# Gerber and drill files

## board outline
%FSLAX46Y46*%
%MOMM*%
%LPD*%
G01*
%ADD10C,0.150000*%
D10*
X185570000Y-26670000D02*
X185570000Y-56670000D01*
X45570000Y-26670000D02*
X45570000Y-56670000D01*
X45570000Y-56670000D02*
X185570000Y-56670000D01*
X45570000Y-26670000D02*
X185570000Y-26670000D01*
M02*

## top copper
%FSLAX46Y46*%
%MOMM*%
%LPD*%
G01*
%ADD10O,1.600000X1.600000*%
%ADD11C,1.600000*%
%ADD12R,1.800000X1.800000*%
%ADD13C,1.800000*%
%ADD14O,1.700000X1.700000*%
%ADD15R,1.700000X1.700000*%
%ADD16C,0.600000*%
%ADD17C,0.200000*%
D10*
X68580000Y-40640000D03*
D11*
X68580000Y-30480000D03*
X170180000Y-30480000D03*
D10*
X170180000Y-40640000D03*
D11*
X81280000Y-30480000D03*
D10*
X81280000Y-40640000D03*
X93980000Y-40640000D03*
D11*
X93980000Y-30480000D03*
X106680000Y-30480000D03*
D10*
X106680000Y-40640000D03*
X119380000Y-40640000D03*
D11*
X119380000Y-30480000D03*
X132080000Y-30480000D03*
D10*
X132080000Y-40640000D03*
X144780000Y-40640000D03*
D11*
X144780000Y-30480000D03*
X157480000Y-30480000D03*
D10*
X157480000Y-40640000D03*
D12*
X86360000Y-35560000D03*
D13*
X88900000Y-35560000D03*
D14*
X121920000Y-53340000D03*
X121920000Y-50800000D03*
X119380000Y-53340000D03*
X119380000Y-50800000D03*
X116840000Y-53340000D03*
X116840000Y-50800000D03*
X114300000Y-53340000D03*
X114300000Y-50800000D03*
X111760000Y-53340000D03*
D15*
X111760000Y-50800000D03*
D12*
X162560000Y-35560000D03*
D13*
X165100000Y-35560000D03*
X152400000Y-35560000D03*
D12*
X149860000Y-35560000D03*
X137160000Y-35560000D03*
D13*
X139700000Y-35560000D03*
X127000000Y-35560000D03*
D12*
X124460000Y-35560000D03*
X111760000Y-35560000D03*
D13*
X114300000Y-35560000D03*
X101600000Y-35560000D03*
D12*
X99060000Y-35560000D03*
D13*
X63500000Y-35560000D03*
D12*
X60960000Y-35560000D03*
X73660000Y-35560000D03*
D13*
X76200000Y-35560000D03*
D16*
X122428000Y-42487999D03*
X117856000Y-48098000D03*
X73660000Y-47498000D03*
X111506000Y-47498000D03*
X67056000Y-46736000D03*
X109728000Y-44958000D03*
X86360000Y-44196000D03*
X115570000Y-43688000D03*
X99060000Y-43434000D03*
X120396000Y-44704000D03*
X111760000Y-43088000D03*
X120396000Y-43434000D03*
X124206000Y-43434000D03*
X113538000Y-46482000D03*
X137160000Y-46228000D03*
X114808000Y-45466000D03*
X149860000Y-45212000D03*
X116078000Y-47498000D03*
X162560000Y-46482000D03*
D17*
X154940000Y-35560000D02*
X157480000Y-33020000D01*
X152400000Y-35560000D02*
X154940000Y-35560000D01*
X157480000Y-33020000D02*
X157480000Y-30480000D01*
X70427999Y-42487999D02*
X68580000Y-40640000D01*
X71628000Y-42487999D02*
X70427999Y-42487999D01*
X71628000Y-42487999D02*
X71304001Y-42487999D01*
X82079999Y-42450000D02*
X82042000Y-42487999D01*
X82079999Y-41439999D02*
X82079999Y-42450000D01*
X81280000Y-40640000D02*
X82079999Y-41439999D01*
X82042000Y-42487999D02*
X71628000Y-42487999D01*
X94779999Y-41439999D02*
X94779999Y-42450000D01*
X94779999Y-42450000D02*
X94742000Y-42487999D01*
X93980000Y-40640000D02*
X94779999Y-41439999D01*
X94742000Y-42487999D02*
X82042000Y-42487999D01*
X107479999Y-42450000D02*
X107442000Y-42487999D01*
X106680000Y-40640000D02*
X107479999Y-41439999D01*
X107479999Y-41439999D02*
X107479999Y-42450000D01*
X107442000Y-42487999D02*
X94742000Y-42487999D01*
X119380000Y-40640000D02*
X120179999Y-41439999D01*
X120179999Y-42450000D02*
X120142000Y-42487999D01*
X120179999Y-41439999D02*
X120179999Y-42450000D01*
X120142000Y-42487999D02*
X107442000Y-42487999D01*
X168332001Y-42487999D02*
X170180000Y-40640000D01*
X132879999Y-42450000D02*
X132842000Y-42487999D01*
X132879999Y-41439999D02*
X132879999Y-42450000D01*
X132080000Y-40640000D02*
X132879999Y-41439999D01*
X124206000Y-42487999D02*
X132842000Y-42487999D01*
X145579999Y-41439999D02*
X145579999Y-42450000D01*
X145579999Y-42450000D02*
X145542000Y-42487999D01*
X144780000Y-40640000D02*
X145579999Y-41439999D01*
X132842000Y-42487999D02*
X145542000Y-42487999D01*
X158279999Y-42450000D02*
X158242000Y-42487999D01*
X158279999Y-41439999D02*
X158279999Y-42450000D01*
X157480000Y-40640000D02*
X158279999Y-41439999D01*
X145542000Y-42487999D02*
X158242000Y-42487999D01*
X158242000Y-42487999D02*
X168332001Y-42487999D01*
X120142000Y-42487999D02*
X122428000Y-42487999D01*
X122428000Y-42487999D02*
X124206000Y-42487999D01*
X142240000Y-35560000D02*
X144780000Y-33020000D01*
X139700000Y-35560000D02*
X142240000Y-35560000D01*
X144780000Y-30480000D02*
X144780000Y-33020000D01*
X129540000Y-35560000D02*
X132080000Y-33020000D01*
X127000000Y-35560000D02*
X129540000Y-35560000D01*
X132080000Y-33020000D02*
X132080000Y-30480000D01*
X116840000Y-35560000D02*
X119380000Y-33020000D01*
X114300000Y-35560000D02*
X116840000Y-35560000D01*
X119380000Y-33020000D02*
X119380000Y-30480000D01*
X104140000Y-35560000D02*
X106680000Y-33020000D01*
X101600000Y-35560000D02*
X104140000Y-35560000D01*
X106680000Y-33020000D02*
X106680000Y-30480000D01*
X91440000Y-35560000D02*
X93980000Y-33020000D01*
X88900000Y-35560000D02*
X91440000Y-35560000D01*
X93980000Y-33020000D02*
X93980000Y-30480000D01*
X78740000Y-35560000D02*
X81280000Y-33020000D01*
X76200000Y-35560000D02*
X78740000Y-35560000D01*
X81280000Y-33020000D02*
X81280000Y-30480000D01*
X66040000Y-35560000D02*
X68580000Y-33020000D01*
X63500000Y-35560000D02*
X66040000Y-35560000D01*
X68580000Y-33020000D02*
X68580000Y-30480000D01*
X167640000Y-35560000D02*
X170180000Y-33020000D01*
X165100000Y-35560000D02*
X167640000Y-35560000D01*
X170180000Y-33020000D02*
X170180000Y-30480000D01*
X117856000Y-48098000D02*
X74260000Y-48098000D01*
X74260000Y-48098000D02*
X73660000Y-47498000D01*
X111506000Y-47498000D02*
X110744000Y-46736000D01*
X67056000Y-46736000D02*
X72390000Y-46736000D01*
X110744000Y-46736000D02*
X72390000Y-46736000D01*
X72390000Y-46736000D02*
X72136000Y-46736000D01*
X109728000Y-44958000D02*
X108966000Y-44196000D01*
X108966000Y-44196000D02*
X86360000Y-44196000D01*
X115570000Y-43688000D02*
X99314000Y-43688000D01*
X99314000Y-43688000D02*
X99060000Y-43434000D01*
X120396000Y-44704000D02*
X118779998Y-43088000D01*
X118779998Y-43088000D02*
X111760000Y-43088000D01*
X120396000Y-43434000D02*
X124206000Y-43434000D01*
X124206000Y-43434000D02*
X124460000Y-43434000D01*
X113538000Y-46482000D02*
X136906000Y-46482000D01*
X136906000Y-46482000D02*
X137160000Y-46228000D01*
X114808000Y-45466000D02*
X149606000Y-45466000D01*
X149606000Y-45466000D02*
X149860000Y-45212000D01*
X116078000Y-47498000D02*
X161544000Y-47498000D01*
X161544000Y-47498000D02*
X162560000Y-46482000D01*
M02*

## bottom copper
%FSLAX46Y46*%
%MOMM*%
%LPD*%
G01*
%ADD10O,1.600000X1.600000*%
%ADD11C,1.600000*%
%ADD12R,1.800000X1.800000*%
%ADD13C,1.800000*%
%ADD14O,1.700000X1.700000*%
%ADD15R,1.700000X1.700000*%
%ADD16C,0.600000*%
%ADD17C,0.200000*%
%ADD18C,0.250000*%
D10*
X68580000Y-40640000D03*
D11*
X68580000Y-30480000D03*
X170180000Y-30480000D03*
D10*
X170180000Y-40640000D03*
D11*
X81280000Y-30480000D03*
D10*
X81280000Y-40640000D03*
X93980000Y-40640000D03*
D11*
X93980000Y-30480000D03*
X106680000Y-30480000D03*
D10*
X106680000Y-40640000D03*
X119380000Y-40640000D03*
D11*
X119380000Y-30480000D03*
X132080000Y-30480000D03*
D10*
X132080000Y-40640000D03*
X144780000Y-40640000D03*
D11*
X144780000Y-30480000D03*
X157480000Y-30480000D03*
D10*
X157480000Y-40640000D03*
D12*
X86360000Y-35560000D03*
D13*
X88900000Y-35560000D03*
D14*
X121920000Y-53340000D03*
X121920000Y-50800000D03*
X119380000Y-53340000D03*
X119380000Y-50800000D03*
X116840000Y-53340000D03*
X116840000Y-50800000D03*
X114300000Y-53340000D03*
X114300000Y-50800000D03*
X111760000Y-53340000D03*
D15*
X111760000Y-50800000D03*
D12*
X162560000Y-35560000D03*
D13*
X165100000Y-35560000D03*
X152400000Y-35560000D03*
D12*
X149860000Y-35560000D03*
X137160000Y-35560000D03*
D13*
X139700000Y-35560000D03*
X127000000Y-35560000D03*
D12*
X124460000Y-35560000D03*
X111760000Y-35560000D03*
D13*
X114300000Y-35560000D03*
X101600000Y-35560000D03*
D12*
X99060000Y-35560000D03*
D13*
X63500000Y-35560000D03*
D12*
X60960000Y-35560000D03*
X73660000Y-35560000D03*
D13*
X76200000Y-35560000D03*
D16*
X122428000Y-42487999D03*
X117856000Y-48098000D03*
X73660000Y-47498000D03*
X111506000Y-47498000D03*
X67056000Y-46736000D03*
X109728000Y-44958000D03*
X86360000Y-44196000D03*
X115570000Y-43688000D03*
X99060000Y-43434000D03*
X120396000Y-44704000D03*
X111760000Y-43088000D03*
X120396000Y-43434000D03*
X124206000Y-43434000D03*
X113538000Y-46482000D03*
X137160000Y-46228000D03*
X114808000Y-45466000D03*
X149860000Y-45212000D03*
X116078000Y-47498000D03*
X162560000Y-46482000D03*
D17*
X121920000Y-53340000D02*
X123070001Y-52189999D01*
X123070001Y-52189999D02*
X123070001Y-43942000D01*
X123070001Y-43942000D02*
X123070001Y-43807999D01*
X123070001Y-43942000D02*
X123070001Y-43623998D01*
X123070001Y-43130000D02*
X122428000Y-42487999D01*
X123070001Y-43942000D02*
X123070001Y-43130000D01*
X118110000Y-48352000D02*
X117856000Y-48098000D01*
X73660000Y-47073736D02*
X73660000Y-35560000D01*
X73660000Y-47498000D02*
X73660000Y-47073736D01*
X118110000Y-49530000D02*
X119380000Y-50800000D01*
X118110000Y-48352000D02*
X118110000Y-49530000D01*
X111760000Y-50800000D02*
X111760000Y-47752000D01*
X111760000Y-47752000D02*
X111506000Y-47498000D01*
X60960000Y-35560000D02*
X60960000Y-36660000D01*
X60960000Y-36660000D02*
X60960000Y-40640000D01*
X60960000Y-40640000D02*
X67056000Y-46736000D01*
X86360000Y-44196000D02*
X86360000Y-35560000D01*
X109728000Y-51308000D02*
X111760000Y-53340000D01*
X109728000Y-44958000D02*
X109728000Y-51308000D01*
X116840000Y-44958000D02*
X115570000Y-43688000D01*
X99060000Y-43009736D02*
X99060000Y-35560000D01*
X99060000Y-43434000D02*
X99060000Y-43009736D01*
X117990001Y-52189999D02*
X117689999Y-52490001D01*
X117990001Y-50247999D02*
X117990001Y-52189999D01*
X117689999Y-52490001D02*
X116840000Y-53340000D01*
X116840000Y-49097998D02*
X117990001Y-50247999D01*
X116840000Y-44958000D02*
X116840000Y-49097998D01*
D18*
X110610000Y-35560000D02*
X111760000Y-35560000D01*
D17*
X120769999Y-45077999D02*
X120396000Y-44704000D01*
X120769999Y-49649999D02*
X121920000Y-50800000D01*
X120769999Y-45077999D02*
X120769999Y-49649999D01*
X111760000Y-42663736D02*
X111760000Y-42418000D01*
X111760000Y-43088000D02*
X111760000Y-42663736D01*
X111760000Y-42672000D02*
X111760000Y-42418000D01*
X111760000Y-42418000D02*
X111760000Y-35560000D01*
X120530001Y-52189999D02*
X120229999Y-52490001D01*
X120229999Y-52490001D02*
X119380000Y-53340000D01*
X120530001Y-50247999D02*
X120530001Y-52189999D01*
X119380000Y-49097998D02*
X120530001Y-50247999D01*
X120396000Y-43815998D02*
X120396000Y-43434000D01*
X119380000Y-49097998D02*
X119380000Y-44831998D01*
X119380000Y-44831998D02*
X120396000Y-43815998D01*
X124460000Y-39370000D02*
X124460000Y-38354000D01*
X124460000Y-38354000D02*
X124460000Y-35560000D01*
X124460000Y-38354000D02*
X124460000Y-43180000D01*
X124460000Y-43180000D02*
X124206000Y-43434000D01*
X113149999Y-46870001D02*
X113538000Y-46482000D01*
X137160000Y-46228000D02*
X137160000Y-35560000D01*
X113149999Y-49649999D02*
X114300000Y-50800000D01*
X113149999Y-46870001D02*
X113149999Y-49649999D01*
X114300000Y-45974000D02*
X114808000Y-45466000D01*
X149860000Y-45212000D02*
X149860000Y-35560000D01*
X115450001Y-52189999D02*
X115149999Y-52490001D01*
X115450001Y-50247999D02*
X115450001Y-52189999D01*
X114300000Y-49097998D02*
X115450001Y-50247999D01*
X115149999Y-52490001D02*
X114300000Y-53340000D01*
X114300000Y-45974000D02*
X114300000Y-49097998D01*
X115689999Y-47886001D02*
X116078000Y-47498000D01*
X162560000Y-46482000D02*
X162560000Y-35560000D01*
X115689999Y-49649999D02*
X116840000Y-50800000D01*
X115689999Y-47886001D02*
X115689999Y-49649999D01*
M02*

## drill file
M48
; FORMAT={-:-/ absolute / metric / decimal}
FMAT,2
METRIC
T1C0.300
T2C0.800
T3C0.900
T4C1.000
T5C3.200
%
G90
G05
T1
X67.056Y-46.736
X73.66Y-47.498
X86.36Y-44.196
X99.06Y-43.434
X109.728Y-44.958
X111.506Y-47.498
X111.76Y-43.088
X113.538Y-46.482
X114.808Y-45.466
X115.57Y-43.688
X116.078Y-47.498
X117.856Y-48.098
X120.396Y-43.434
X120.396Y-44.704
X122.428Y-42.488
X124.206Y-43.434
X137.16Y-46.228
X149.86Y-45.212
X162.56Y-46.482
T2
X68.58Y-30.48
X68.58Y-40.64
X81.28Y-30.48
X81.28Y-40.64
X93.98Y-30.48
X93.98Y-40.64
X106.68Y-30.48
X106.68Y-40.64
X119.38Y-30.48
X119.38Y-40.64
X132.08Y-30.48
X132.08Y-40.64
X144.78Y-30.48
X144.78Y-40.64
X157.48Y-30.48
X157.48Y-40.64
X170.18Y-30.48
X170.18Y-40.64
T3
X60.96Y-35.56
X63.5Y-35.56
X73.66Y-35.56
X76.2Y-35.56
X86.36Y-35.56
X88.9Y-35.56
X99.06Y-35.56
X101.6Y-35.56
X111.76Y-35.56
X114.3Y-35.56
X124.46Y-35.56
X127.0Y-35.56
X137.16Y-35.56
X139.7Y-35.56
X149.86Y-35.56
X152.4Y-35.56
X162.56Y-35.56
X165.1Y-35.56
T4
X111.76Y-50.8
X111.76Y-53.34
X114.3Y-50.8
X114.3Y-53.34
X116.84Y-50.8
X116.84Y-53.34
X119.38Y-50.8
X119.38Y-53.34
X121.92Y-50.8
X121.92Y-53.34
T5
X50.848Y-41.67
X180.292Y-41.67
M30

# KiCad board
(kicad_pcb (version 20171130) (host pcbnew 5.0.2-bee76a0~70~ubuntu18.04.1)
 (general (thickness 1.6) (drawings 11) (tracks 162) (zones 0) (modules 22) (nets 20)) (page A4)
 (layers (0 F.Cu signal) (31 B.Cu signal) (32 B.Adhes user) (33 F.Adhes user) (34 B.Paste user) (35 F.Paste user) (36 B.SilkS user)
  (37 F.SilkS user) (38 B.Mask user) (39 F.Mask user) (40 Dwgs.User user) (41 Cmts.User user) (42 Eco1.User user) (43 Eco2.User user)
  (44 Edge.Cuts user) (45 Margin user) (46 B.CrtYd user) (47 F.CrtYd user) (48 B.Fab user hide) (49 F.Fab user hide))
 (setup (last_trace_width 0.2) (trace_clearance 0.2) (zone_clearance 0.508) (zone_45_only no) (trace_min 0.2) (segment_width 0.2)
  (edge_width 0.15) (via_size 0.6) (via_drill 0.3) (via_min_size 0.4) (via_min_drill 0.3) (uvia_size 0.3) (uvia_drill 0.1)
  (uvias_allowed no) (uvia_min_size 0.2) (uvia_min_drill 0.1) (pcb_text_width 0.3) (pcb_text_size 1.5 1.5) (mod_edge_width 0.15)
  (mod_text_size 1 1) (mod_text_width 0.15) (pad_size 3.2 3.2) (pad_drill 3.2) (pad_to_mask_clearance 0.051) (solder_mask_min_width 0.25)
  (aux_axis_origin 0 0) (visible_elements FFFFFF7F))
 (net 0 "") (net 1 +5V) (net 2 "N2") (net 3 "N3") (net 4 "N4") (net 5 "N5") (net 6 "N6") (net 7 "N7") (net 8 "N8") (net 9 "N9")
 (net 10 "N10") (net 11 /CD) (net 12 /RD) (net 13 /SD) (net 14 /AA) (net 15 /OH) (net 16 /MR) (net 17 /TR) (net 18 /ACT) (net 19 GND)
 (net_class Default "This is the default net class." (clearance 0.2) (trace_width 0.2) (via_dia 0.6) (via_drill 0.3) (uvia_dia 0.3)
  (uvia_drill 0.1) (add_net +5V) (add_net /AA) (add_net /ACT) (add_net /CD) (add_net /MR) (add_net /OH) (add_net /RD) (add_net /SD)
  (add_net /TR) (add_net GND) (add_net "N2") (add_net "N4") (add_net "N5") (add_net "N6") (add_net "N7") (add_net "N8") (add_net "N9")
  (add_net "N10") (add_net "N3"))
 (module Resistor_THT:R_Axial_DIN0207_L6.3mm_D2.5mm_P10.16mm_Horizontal (layer F.Cu) (at 68.58 30.48 270)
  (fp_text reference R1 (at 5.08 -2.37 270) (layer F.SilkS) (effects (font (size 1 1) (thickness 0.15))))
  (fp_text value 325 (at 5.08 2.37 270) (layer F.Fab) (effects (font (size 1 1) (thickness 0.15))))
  (pad 2 thru_hole oval (at 10.16 0 270) (size 1.6 1.6) (drill 0.8) (layers *.Cu *.Mask) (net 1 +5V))
  (pad 1 thru_hole circle (at 0 0 270) (size 1.6 1.6) (drill 0.8) (layers *.Cu *.Mask) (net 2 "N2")))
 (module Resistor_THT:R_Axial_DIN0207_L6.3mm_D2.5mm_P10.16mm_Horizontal (layer F.Cu) (at 170.18 30.48 270)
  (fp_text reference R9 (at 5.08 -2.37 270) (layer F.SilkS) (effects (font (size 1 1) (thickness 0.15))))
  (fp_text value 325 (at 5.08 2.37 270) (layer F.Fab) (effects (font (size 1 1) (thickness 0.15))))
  (pad 1 thru_hole circle (at 0 0 270) (size 1.6 1.6) (drill 0.8) (layers *.Cu *.Mask) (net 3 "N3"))
  (pad 2 thru_hole oval (at 10.16 0 270) (size 1.6 1.6) (drill 0.8) (layers *.Cu *.Mask) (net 1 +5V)))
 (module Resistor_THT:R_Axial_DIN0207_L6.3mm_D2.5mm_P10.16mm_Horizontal (layer F.Cu) (at 81.28 30.48 270)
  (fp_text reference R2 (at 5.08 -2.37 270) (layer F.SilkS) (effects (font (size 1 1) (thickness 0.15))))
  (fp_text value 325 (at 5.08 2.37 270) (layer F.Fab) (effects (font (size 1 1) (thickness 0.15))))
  (pad 1 thru_hole circle (at 0 0 270) (size 1.6 1.6) (drill 0.8) (layers *.Cu *.Mask) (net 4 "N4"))
  (pad 2 thru_hole oval (at 10.16 0 270) (size 1.6 1.6) (drill 0.8) (layers *.Cu *.Mask) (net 1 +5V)))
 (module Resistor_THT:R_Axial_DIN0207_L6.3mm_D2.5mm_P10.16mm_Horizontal (layer F.Cu) (at 93.98 30.48 270)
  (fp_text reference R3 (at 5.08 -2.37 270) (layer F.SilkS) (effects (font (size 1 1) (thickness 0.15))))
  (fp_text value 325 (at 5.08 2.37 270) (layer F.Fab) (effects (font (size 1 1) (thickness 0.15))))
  (pad 2 thru_hole oval (at 10.16 0 270) (size 1.6 1.6) (drill 0.8) (layers *.Cu *.Mask) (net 1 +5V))
  (pad 1 thru_hole circle (at 0 0 270) (size 1.6 1.6) (drill 0.8) (layers *.Cu *.Mask) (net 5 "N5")))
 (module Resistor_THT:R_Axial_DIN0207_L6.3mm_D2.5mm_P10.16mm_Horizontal (layer F.Cu) (at 106.68 30.48 270)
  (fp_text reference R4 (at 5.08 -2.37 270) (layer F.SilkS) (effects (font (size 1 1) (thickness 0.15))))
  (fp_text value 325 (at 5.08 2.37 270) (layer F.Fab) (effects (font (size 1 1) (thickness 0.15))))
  (pad 1 thru_hole circle (at 0 0 270) (size 1.6 1.6) (drill 0.8) (layers *.Cu *.Mask) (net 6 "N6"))
  (pad 2 thru_hole oval (at 10.16 0 270) (size 1.6 1.6) (drill 0.8) (layers *.Cu *.Mask) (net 1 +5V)))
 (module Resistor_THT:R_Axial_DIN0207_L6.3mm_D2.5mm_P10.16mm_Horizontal (layer F.Cu) (at 119.38 30.48 270)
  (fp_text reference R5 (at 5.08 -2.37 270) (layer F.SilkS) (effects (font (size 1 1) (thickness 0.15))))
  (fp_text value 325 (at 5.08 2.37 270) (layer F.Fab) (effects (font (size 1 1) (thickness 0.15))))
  (pad 2 thru_hole oval (at 10.16 0 270) (size 1.6 1.6) (drill 0.8) (layers *.Cu *.Mask) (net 1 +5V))
  (pad 1 thru_hole circle (at 0 0 270) (size 1.6 1.6) (drill 0.8) (layers *.Cu *.Mask) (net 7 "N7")))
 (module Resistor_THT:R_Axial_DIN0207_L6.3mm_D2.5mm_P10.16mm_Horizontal (layer F.Cu) (at 132.08 30.48 270)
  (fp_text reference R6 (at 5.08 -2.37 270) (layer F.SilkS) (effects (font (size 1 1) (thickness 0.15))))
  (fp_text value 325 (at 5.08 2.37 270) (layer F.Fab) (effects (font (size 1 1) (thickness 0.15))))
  (pad 1 thru_hole circle (at 0 0 270) (size 1.6 1.6) (drill 0.8) (layers *.Cu *.Mask) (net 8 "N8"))
  (pad 2 thru_hole oval (at 10.16 0 270) (size 1.6 1.6) (drill 0.8) (layers *.Cu *.Mask) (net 1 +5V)))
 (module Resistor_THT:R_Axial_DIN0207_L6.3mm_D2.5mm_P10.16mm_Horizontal (layer F.Cu) (at 144.78 30.48 270)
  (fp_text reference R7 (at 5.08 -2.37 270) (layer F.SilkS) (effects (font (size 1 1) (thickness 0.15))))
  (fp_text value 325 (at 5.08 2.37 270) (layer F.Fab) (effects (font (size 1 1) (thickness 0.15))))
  (pad 2 thru_hole oval (at 10.16 0 270) (size 1.6 1.6) (drill 0.8) (layers *.Cu *.Mask) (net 1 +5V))
  (pad 1 thru_hole circle (at 0 0 270) (size 1.6 1.6) (drill 0.8) (layers *.Cu *.Mask) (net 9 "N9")))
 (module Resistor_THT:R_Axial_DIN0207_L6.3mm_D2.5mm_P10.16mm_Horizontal (layer F.Cu) (at 157.48 30.48 270)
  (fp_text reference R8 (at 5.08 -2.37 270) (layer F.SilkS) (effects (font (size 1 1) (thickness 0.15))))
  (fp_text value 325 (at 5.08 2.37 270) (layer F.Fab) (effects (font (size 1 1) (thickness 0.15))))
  (pad 1 thru_hole circle (at 0 0 270) (size 1.6 1.6) (drill 0.8) (layers *.Cu *.Mask) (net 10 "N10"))
  (pad 2 thru_hole oval (at 10.16 0 270) (size 1.6 1.6) (drill 0.8) (layers *.Cu *.Mask) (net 1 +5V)))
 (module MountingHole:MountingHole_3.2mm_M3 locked (layer F.Cu) (at 180.292 41.67)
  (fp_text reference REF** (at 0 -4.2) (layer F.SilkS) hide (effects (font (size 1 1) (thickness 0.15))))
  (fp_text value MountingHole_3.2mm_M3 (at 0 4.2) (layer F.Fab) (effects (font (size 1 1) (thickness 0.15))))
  (pad 1 np_thru_hole circle (at 0 0) (size 3.2 3.2) (drill 3.2) (layers *.Cu *.Mask)))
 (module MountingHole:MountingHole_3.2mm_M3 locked (layer F.Cu) (at 50.848 41.67)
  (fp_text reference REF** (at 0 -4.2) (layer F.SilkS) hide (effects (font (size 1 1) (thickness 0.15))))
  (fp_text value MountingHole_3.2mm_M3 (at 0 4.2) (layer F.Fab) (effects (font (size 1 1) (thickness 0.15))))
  (pad 1 np_thru_hole circle (at 0 0) (size 3.2 3.2) (drill 3.2) (layers *.Cu *.Mask)))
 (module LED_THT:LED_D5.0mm (layer F.Cu) (at 86.36 35.56)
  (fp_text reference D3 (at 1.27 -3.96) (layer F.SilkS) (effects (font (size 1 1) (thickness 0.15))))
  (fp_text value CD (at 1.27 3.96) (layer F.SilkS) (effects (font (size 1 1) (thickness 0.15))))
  (pad 1 thru_hole rect (at 0 0) (size 1.8 1.8) (drill 0.9) (layers *.Cu *.Mask) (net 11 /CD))
  (pad 2 thru_hole circle (at 2.54 0) (size 1.8 1.8) (drill 0.9) (layers *.Cu *.Mask) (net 5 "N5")))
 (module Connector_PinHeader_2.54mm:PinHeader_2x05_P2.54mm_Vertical (layer B.Cu) (at 111.76 50.8 270)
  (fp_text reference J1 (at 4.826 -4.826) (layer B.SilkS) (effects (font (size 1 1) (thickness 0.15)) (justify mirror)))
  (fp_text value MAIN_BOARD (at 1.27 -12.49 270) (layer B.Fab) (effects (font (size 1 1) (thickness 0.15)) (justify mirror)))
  (pad 10 thru_hole oval (at 2.54 -10.16 270) (size 1.7 1.7) (drill 1) (layers *.Cu *.Mask) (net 1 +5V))
  (pad 9 thru_hole oval (at 0 -10.16 270) (size 1.7 1.7) (drill 1) (layers *.Cu *.Mask) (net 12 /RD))
  (pad 8 thru_hole oval (at 2.54 -7.62 270) (size 1.7 1.7) (drill 1) (layers *.Cu *.Mask) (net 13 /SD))
  (pad 7 thru_hole oval (at 0 -7.62 270) (size 1.7 1.7) (drill 1) (layers *.Cu *.Mask) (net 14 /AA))
  (pad 6 thru_hole oval (at 2.54 -5.08 270) (size 1.7 1.7) (drill 1) (layers *.Cu *.Mask) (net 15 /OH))
  (pad 5 thru_hole oval (at 0 -5.08 270) (size 1.7 1.7) (drill 1) (layers *.Cu *.Mask) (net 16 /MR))
  (pad 4 thru_hole oval (at 2.54 -2.54 270) (size 1.7 1.7) (drill 1) (layers *.Cu *.Mask) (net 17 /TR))
  (pad 3 thru_hole oval (at 0 -2.54 270) (size 1.7 1.7) (drill 1) (layers *.Cu *.Mask) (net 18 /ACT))
  (pad 2 thru_hole oval (at 2.54 0 270) (size 1.7 1.7) (drill 1) (layers *.Cu *.Mask) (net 11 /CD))
  (pad 1 thru_hole rect (at 0 0 270) (size 1.7 1.7) (drill 1) (layers *.Cu *.Mask) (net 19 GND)))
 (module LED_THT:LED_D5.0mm (layer F.Cu) (at 162.56 35.56)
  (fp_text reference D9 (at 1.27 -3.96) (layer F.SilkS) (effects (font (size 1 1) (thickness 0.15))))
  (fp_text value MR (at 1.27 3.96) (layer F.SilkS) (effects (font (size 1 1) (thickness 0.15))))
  (pad 1 thru_hole rect (at 0 0) (size 1.8 1.8) (drill 0.9) (layers *.Cu *.Mask) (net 16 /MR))
  (pad 2 thru_hole circle (at 2.54 0) (size 1.8 1.8) (drill 0.9) (layers *.Cu *.Mask) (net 3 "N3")))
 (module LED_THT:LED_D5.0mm (layer F.Cu) (at 149.86 35.56)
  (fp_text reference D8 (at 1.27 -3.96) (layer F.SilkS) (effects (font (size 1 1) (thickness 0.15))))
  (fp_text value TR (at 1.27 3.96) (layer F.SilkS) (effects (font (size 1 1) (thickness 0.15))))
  (pad 2 thru_hole circle (at 2.54 0) (size 1.8 1.8) (drill 0.9) (layers *.Cu *.Mask) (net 10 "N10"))
  (pad 1 thru_hole rect (at 0 0) (size 1.8 1.8) (drill 0.9) (layers *.Cu *.Mask) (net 17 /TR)))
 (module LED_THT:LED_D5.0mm (layer F.Cu) (at 137.16 35.56)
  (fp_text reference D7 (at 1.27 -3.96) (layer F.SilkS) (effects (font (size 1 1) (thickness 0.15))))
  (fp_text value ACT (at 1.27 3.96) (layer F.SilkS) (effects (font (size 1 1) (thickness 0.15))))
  (pad 1 thru_hole rect (at 0 0) (size 1.8 1.8) (drill 0.9) (layers *.Cu *.Mask) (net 18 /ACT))
  (pad 2 thru_hole circle (at 2.54 0) (size 1.8 1.8) (drill 0.9) (layers *.Cu *.Mask) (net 9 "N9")))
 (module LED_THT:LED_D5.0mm (layer F.Cu) (at 124.46 35.56)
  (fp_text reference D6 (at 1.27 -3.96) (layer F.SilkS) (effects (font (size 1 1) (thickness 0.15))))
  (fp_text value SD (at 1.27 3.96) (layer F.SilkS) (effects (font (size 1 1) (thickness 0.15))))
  (pad 2 thru_hole circle (at 2.54 0) (size 1.8 1.8) (drill 0.9) (layers *.Cu *.Mask) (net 8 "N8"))
  (pad 1 thru_hole rect (at 0 0) (size 1.8 1.8) (drill 0.9) (layers *.Cu *.Mask) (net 13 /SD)))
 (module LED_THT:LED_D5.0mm (layer F.Cu) (at 111.76 35.56)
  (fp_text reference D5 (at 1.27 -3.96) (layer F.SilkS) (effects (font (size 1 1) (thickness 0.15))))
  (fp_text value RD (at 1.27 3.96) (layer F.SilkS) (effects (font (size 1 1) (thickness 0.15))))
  (pad 1 thru_hole rect (at 0 0) (size 1.8 1.8) (drill 0.9) (layers *.Cu *.Mask) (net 12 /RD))
  (pad 2 thru_hole circle (at 2.54 0) (size 1.8 1.8) (drill 0.9) (layers *.Cu *.Mask) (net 7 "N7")))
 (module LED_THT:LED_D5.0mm (layer F.Cu) (at 99.06 35.56)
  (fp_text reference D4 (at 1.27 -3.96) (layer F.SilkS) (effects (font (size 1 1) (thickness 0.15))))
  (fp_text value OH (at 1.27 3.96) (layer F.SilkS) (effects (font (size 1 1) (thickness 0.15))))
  (pad 2 thru_hole circle (at 2.54 0) (size 1.8 1.8) (drill 0.9) (layers *.Cu *.Mask) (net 6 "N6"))
  (pad 1 thru_hole rect (at 0 0) (size 1.8 1.8) (drill 0.9) (layers *.Cu *.Mask) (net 15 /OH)))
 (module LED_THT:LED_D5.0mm (layer F.Cu) (at 60.96 35.56)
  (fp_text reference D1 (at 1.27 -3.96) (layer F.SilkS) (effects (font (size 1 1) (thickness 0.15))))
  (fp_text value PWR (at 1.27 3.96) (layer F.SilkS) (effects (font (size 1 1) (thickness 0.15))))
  (pad 2 thru_hole circle (at 2.54 0) (size 1.8 1.8) (drill 0.9) (layers *.Cu *.Mask) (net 2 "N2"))
  (pad 1 thru_hole rect (at 0 0) (size 1.8 1.8) (drill 0.9) (layers *.Cu *.Mask) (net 19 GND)))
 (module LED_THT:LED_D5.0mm (layer F.Cu) (at 73.66 35.56)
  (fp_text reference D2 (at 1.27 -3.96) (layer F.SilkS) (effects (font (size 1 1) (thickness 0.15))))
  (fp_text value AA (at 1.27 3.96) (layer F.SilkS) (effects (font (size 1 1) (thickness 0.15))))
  (pad 1 thru_hole rect (at 0 0) (size 1.8 1.8) (drill 0.9) (layers *.Cu *.Mask) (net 14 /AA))
  (pad 2 thru_hole circle (at 2.54 0) (size 1.8 1.8) (drill 0.9) (layers *.Cu *.Mask) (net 4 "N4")))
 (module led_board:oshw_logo (layer F.Cu) (at 51.01 50.8)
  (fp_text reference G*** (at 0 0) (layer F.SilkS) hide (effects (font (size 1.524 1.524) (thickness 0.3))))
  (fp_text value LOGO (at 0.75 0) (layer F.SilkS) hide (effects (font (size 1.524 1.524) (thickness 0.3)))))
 (gr_line (start 185.57 26.67) (end 185.57 56.67) (layer Edge.Cuts) (width 0.15))
 (gr_line (start 45.57 26.67) (end 45.57 56.67) (layer Edge.Cuts) (width 0.15))
 (gr_line (start 45.57 56.67) (end 185.57 56.67) (layer Edge.Cuts) (width 0.15))
 (gr_line (start 45.57 26.67) (end 185.57 26.67) (layer Edge.Cuts) (width 0.15))
 (segment (start 154.94 35.56) (end 157.48 33.02) (width 0.2) (layer F.Cu) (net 10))
 (segment (start 152.4 35.56) (end 154.94 35.56) (width 0.2) (layer F.Cu) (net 10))
 (segment (start 157.48 33.02) (end 157.48 30.48) (width 0.2) (layer F.Cu) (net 10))
 (segment (start 121.92 53.34) (end 123.070001 52.189999) (width 0.2) (layer B.Cu) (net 1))
 (segment (start 70.427999 42.487999) (end 68.58 40.64) (width 0.2) (layer F.Cu) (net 1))
 (segment (start 71.628 42.487999) (end 70.427999 42.487999) (width 0.2) (layer F.Cu) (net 1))
 (segment (start 71.628 42.487999) (end 71.304001 42.487999) (width 0.2) (layer F.Cu) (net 1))
 (segment (start 82.079999 42.45) (end 82.042 42.487999) (width 0.2) (layer F.Cu) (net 1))
 (segment (start 82.079999 41.439999) (end 82.079999 42.45) (width 0.2) (layer F.Cu) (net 1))
 (segment (start 81.28 40.64) (end 82.079999 41.439999) (width 0.2) (layer F.Cu) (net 1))
 (segment (start 82.042 42.487999) (end 71.628 42.487999) (width 0.2) (layer F.Cu) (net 1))
 (segment (start 94.779999 41.439999) (end 94.779999 42.45) (width 0.2) (layer F.Cu) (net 1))
 (segment (start 94.779999 42.45) (end 94.742 42.487999) (width 0.2) (layer F.Cu) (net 1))
 (segment (start 93.98 40.64) (end 94.779999 41.439999) (width 0.2) (layer F.Cu) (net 1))
 (segment (start 94.742 42.487999) (end 82.042 42.487999) (width 0.2) (layer F.Cu) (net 1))
 (segment (start 107.479999 42.45) (end 107.442 42.487999) (width 0.2) (layer F.Cu) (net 1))
 (segment (start 106.68 40.64) (end 107.479999 41.439999) (width 0.2) (layer F.Cu) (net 1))
 (segment (start 107.479999 41.439999) (end 107.479999 42.45) (width 0.2) (layer F.Cu) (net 1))
 (segment (start 107.442 42.487999) (end 94.742 42.487999) (width 0.2) (layer F.Cu) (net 1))
 (segment (start 119.38 40.64) (end 120.179999 41.439999) (width 0.2) (layer F.Cu) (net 1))
 (segment (start 120.179999 42.45) (end 120.142 42.487999) (width 0.2) (layer F.Cu) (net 1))
 (segment (start 120.179999 41.439999) (end 120.179999 42.45) (width 0.2) (layer F.Cu) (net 1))
 (segment (start 120.142 42.487999) (end 107.442 42.487999) (width 0.2) (layer F.Cu) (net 1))
 (segment (start 168.332001 42.487999) (end 170.18 40.64) (width 0.2) (layer F.Cu) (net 1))
 (segment (start 123.070001 52.189999) (end 123.070001 43.942) (width 0.2) (layer B.Cu) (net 1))
 (segment (start 123.070001 43.942) (end 123.070001 43.807999) (width 0.2) (layer B.Cu) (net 1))
 (segment (start 123.070001 43.942) (end 123.070001 43.623998) (width 0.2) (layer B.Cu) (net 1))
 (segment (start 132.879999 42.45) (end 132.842 42.487999) (width 0.2) (layer F.Cu) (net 1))
 (segment (start 132.879999 41.439999) (end 132.879999 42.45) (width 0.2) (layer F.Cu) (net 1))
 (segment (start 132.08 40.64) (end 132.879999 41.439999) (width 0.2) (layer F.Cu) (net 1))
 (segment (start 124.206 42.487999) (end 132.842 42.487999) (width 0.2) (layer F.Cu) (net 1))
 (segment (start 145.579999 41.439999) (end 145.579999 42.45) (width 0.2) (layer F.Cu) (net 1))
 (segment (start 145.579999 42.45) (end 145.542 42.487999) (width 0.2) (layer F.Cu) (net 1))
 (segment (start 144.78 40.64) (end 145.579999 41.439999) (width 0.2) (layer F.Cu) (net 1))
 (segment (start 132.842 42.487999) (end 145.542 42.487999) (width 0.2) (layer F.Cu) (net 1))
 (segment (start 158.279999 42.45) (end 158.242 42.487999) (width 0.2) (layer F.Cu) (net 1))
 (segment (start 158.279999 41.439999) (end 158.279999 42.45) (width 0.2) (layer F.Cu) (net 1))
 (segment (start 157.48 40.64) (end 158.279999 41.439999) (width 0.2) (layer F.Cu) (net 1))
 (segment (start 145.542 42.487999) (end 158.242 42.487999) (width 0.2) (layer F.Cu) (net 1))
 (segment (start 158.242 42.487999) (end 168.332001 42.487999) (width 0.2) (layer F.Cu) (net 1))
 (segment (start 123.070001 43.13) (end 122.428 42.487999) (width 0.2) (layer B.Cu) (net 1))
 (segment (start 123.070001 43.942) (end 123.070001 43.13) (width 0.2) (layer B.Cu) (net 1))
 (segment (start 120.142 42.487999) (end 122.428 42.487999) (width 0.2) (layer F.Cu) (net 1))
 (via (at 122.428 42.487999) (size 0.6) (drill 0.3) (layers F.Cu B.Cu) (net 1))
 (segment (start 122.428 42.487999) (end 124.206 42.487999) (width 0.2) (layer F.Cu) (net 1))
 (segment (start 142.24 35.56) (end 144.78 33.02) (width 0.2) (layer F.Cu) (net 9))
 (segment (start 139.7 35.56) (end 142.24 35.56) (width 0.2) (layer F.Cu) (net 9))
 (segment (start 144.78 30.48) (end 144.78 33.02) (width 0.2) (layer F.Cu) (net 9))
 (segment (start 129.54 35.56) (end 132.08 33.02) (width 0.2) (layer F.Cu) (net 8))
 (segment (start 127 35.56) (end 129.54 35.56) (width 0.2) (layer F.Cu) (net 8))
 (segment (start 132.08 33.02) (end 132.08 30.48) (width 0.2) (layer F.Cu) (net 8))
 (segment (start 116.84 35.56) (end 119.38 33.02) (width 0.2) (layer F.Cu) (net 7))
 (segment (start 114.3 35.56) (end 116.84 35.56) (width 0.2) (layer F.Cu) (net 7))
 (segment (start 119.38 33.02) (end 119.38 30.48) (width 0.2) (layer F.Cu) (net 7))
 (segment (start 104.14 35.56) (end 106.68 33.02) (width 0.2) (layer F.Cu) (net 6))
 (segment (start 101.6 35.56) (end 104.14 35.56) (width 0.2) (layer F.Cu) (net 6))
 (segment (start 106.68 33.02) (end 106.68 30.48) (width 0.2) (layer F.Cu) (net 6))
 (segment (start 91.44 35.56) (end 93.98 33.02) (width 0.2) (layer F.Cu) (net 5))
 (segment (start 88.9 35.56) (end 91.44 35.56) (width 0.2) (layer F.Cu) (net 5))
 (segment (start 93.98 33.02) (end 93.98 30.48) (width 0.2) (layer F.Cu) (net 5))
 (segment (start 78.74 35.56) (end 81.28 33.02) (width 0.2) (layer F.Cu) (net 4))
 (segment (start 76.2 35.56) (end 78.74 35.56) (width 0.2) (layer F.Cu) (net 4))
 (segment (start 81.28 33.02) (end 81.28 30.48) (width 0.2) (layer F.Cu) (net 4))
 (segment (start 66.04 35.56) (end 68.58 33.02) (width 0.2) (layer F.Cu) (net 2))
 (segment (start 63.5 35.56) (end 66.04 35.56) (width 0.2) (layer F.Cu) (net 2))
 (segment (start 68.58 33.02) (end 68.58 30.48) (width 0.2) (layer F.Cu) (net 2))
 (segment (start 167.64 35.56) (end 170.18 33.02) (width 0.2) (layer F.Cu) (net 3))
 (segment (start 165.1 35.56) (end 167.64 35.56) (width 0.2) (layer F.Cu) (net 3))
 (segment (start 170.18 33.02) (end 170.18 30.48) (width 0.2) (layer F.Cu) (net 3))
 (via (at 117.856 48.098) (size 0.6) (drill 0.3) (layers F.Cu B.Cu) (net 14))
 (segment (start 118.11 48.352) (end 117.856 48.098) (width 0.2) (layer B.Cu) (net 14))
 (via (at 73.66 47.498) (size 0.6) (drill 0.3) (layers F.Cu B.Cu) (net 14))
 (segment (start 117.856 48.098) (end 74.26 48.098) (width 0.2) (layer F.Cu) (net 14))
 (segment (start 74.26 48.098) (end 73.66 47.498) (width 0.2) (layer F.Cu) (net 14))
 (segment (start 73.66 47.073736) (end 73.66 35.56) (width 0.2) (layer B.Cu) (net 14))
 (segment (start 73.66 47.498) (end 73.66 47.073736) (width 0.2) (layer B.Cu) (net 14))
 (segment (start 118.11 49.53) (end 119.38 50.8) (width 0.2) (layer B.Cu) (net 14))
 (segment (start 118.11 48.352) (end 118.11 49.53) (width 0.2) (layer B.Cu) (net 14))
 (segment (start 111.76 50.8) (end 111.76 47.752) (width 0.2) (layer B.Cu) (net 19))
 (via (at 111.506 47.498) (size 0.6) (drill 0.3) (layers F.Cu B.Cu) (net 19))
 (segment (start 111.76 47.752) (end 111.506 47.498) (width 0.2) (layer B.Cu) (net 19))
 (segment (start 111.506 47.498) (end 110.744 46.736) (width 0.2) (layer F.Cu) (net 19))
 (segment (start 60.96 35.56) (end 60.96 36.66) (width 0.2) (layer B.Cu) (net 19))
 (via (at 67.056 46.736) (size 0.6) (drill 0.3) (layers F.Cu B.Cu) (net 19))
 (segment (start 60.96 36.66) (end 60.96 40.64) (width 0.2) (layer B.Cu) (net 19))
 (segment (start 60.96 40.64) (end 67.056 46.736) (width 0.2) (layer B.Cu) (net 19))
 (segment (start 67.056 46.736) (end 72.39 46.736) (width 0.2) (layer F.Cu) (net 19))
 (segment (start 110.744 46.736) (end 72.39 46.736) (width 0.2) (layer F.Cu) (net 19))
 (segment (start 72.39 46.736) (end 72.136 46.736) (width 0.2) (layer F.Cu) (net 19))
 (via (at 109.728 44.958) (size 0.6) (drill 0.3) (layers F.Cu B.Cu) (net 11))
 (via (at 86.36 44.196) (size 0.6) (drill 0.3) (layers F.Cu B.Cu) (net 11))
 (segment (start 109.728 44.958) (end 108.966 44.196) (width 0.2) (layer F.Cu) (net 11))
 (segment (start 108.966 44.196) (end 86.36 44.196) (width 0.2) (layer F.Cu) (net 11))
 (segment (start 86.36 44.196) (end 86.36 35.56) (width 0.2) (layer B.Cu) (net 11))
 (segment (start 109.728 51.308) (end 111.76 53.34) (width 0.2) (layer B.Cu) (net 11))
 (segment (start 109.728 44.958) (end 109.728 51.308) (width 0.2) (layer B.Cu) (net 11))
 (via (at 115.57 43.688) (size 0.6) (drill 0.3) (layers F.Cu B.Cu) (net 15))
 (segment (start 116.84 44.958) (end 115.57 43.688) (width 0.2) (layer B.Cu) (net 15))
 (via (at 99.06 43.434) (size 0.6) (drill 0.3) (layers F.Cu B.Cu) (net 15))
 (segment (start 115.57 43.688) (end 99.314 43.688) (width 0.2) (layer F.Cu) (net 15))
 (segment (start 99.314 43.688) (end 99.06 43.434) (width 0.2) (layer F.Cu) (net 15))
 (segment (start 99.06 43.009736) (end 99.06 35.56) (width 0.2) (layer B.Cu) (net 15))
 (segment (start 99.06 43.434) (end 99.06 43.009736) (width 0.2) (layer B.Cu) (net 15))
 (segment (start 117.990001 52.189999) (end 117.689999 52.490001) (width 0.2) (layer B.Cu) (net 15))
 (segment (start 117.990001 50.247999) (end 117.990001 52.189999) (width 0.2) (layer B.Cu) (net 15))
 (segment (start 117.689999 52.490001) (end 116.84 53.34) (width 0.2) (layer B.Cu) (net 15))
 (segment (start 116.84 49.097998) (end 117.990001 50.247999) (width 0.2) (layer B.Cu) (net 15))
 (segment (start 116.84 44.958) (end 116.84 49.097998) (width 0.2) (layer B.Cu) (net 15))
 (segment (start 110.61 35.56) (end 111.76 35.56) (width 0.25) (layer B.Cu) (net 12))
 (via (at 120.396 44.704) (size 0.6) (drill 0.3) (layers F.Cu B.Cu) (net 12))
 (segment (start 120.769999 45.077999) (end 120.396 44.704) (width 0.2) (layer B.Cu) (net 12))
 (segment (start 120.769999 49.649999) (end 121.92 50.8) (width 0.2) (layer B.Cu) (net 12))
 (segment (start 120.769999 45.077999) (end 120.769999 49.649999) (width 0.2) (layer B.Cu) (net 12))
 (via (at 111.76 43.088) (size 0.6) (drill 0.3) (layers F.Cu B.Cu) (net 12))
 (segment (start 120.396 44.704) (end 118.779998 43.088) (width 0.2) (layer F.Cu) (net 12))
 (segment (start 118.779998 43.088) (end 111.76 43.088) (width 0.2) (layer F.Cu) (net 12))
 (segment (start 111.76 42.663736) (end 111.76 42.418) (width 0.2) (layer B.Cu) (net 12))
 (segment (start 111.76 43.088) (end 111.76 42.663736) (width 0.2) (layer B.Cu) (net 12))
 (segment (start 111.76 42.672) (end 111.76 42.418) (width 0.2) (layer B.Cu) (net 12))
 (segment (start 111.76 42.418) (end 111.76 35.56) (width 0.2) (layer B.Cu) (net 12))
 (segment (start 120.530001 52.189999) (end 120.229999 52.490001) (width 0.2) (layer B.Cu) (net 13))
 (segment (start 120.229999 52.490001) (end 119.38 53.34) (width 0.2) (layer B.Cu) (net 13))
 (segment (start 120.530001 50.247999) (end 120.530001 52.189999) (width 0.2) (layer B.Cu) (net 13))
 (segment (start 119.38 49.097998) (end 120.530001 50.247999) (width 0.2) (layer B.Cu) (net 13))
 (segment (start 120.396 43.815998) (end 120.396 43.434) (width 0.2) (layer B.Cu) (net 13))
 (via (at 120.396 43.434) (size 0.6) (drill 0.3) (layers F.Cu B.Cu) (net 13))
 (segment (start 119.38 49.097998) (end 119.38 44.831998) (width 0.2) (layer B.Cu) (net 13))
 (segment (start 119.38 44.831998) (end 120.396 43.815998) (width 0.2) (layer B.Cu) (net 13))
 (via (at 124.206 43.434) (size 0.6) (drill 0.3) (layers F.Cu B.Cu) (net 13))
 (segment (start 124.46 39.37) (end 124.46 38.354) (width 0.2) (layer B.Cu) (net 13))
 (segment (start 124.46 38.354) (end 124.46 35.56) (width 0.2) (layer B.Cu) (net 13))
 (segment (start 120.396 43.434) (end 124.206 43.434) (width 0.2) (layer F.Cu) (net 13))
 (segment (start 124.46 38.354) (end 124.46 43.18) (width 0.2) (layer B.Cu) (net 13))
 (segment (start 124.206 43.434) (end 124.46 43.434) (width 0.2) (layer F.Cu) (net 13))
 (segment (start 124.46 43.18) (end 124.206 43.434) (width 0.2) (layer B.Cu) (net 13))
 (via (at 113.538 46.482) (size 0.6) (drill 0.3) (layers F.Cu B.Cu) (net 18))
 (segment (start 113.149999 46.870001) (end 113.538 46.482) (width 0.2) (layer B.Cu) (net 18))
 (via (at 137.16 46.228) (size 0.6) (drill 0.3) (layers F.Cu B.Cu) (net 18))
 (segment (start 113.538 46.482) (end 136.906 46.482) (width 0.2) (layer F.Cu) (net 18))
 (segment (start 136.906 46.482) (end 137.16 46.228) (width 0.2) (layer F.Cu) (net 18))
 (segment (start 137.16 46.228) (end 137.16 35.56) (width 0.2) (layer B.Cu) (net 18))
 (segment (start 113.149999 49.649999) (end 114.3 50.8) (width 0.2) (layer B.Cu) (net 18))
 (segment (start 113.149999 46.870001) (end 113.149999 49.649999) (width 0.2) (layer B.Cu) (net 18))
 (via (at 114.808 45.466) (size 0.6) (drill 0.3) (layers F.Cu B.Cu) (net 17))
 (segment (start 114.3 45.974) (end 114.808 45.466) (width 0.2) (layer B.Cu) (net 17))
 (via (at 149.86 45.212) (size 0.6) (drill 0.3) (layers F.Cu B.Cu) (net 17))
 (segment (start 114.808 45.466) (end 149.606 45.466) (width 0.2) (layer F.Cu) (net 17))
 (segment (start 149.606 45.466) (end 149.86 45.212) (width 0.2) (layer F.Cu) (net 17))
 (segment (start 149.86 45.212) (end 149.86 35.56) (width 0.2) (layer B.Cu) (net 17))
 (segment (start 115.450001 52.189999) (end 115.149999 52.490001) (width 0.2) (layer B.Cu) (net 17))
 (segment (start 115.450001 50.247999) (end 115.450001 52.189999) (width 0.2) (layer B.Cu) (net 17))
 (segment (start 114.3 49.097998) (end 115.450001 50.247999) (width 0.2) (layer B.Cu) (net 17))
 (segment (start 115.149999 52.490001) (end 114.3 53.34) (width 0.2) (layer B.Cu) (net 17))
 (segment (start 114.3 45.974) (end 114.3 49.097998) (width 0.2) (layer B.Cu) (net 17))
 (segment (start 115.689999 47.886001) (end 116.078 47.498) (width 0.2) (layer B.Cu) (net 16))
 (via (at 116.078 47.498) (size 0.6) (drill 0.3) (layers F.Cu B.Cu) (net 16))
 (via (at 162.56 46.482) (size 0.6) (drill 0.3) (layers F.Cu B.Cu) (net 16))
 (segment (start 116.078 47.498) (end 161.544 47.498) (width 0.2) (layer F.Cu) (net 16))
 (segment (start 161.544 47.498) (end 162.56 46.482) (width 0.2) (layer F.Cu) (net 16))
 (segment (start 162.56 46.482) (end 162.56 35.56) (width 0.2) (layer B.Cu) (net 16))
 (segment (start 115.689999 49.649999) (end 116.84 50.8) (width 0.2) (layer B.Cu) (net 16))
 (segment (start 115.689999 47.886001) (end 115.689999 49.649999) (width 0.2) (layer B.Cu) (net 16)))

